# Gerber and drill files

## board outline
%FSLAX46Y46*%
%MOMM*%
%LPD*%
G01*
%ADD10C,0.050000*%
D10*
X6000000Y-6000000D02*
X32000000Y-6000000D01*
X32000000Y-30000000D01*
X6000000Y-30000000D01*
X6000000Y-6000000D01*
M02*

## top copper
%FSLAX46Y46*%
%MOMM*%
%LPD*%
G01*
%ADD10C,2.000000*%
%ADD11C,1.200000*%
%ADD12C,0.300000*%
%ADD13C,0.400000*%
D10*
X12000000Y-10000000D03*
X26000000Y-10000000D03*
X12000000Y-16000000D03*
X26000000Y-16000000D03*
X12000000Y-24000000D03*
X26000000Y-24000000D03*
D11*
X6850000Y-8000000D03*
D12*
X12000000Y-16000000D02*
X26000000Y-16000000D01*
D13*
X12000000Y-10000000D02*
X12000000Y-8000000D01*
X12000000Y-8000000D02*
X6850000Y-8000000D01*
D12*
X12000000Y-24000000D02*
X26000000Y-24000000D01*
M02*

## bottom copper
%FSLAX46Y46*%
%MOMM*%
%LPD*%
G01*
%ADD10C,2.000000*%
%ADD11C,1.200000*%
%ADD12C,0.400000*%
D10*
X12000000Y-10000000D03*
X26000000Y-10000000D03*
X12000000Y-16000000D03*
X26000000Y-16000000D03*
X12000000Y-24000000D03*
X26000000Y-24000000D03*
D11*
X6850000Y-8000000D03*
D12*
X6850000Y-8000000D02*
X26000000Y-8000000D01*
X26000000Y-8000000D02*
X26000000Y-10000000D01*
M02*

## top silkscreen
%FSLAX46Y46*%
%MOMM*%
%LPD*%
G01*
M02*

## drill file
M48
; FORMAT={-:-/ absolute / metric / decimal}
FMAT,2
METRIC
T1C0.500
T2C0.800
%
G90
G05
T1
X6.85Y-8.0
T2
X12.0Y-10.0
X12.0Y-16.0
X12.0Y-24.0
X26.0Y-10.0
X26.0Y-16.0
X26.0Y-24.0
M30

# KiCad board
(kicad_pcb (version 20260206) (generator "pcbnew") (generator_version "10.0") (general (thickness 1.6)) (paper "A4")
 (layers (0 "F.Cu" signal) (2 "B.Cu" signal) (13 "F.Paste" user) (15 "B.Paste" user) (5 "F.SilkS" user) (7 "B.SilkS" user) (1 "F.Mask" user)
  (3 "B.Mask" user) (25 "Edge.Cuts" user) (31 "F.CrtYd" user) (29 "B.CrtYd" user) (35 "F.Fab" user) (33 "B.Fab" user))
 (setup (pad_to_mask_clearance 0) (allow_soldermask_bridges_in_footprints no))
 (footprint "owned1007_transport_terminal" (layer "F.Cu") (at 12 10)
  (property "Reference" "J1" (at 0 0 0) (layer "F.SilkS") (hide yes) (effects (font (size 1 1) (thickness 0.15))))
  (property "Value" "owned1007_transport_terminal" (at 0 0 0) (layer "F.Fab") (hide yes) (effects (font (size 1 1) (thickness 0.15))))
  (pad "1" thru_hole circle (at 0 0) (size 2 2) (drill 0.8) (layers "*.Cu" "*.Mask") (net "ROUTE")))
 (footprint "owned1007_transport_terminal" (layer "F.Cu") (at 26 10)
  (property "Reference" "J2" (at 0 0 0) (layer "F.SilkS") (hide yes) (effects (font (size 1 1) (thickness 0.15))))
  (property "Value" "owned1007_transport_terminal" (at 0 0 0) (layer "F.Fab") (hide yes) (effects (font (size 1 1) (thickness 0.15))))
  (pad "1" thru_hole circle (at 0 0) (size 2 2) (drill 0.8) (layers "*.Cu" "*.Mask") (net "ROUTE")))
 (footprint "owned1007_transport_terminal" (layer "F.Cu") (at 12 16)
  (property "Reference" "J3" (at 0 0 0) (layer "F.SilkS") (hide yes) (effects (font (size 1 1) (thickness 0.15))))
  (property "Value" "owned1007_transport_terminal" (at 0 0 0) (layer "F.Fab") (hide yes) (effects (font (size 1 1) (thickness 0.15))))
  (pad "1" thru_hole circle (at 0 0) (size 2 2) (drill 0.8) (layers "*.Cu" "*.Mask") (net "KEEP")))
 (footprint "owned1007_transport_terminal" (layer "F.Cu") (at 26 16)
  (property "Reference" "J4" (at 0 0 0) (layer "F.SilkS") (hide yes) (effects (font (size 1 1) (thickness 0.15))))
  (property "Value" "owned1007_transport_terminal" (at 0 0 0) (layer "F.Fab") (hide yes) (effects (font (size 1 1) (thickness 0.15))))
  (pad "1" thru_hole circle (at 0 0) (size 2 2) (drill 0.8) (layers "*.Cu" "*.Mask") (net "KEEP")))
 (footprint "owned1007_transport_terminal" (layer "F.Cu") (at 12 24)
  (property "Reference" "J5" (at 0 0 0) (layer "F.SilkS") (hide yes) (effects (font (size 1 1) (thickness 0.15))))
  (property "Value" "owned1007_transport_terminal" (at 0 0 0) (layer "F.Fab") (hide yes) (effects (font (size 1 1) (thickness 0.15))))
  (pad "1" thru_hole circle (at 0 0) (size 2 2) (drill 0.8) (layers "*.Cu" "*.Mask") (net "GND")))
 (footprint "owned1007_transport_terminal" (layer "F.Cu") (at 26 24)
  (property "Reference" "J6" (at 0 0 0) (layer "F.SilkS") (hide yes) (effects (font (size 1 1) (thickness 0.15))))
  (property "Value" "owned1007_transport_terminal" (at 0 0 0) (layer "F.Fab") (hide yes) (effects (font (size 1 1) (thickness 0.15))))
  (pad "1" thru_hole circle (at 0 0) (size 2 2) (drill 0.8) (layers "*.Cu" "*.Mask") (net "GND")))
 (gr_rect (start 6 6) (end 32 30) (stroke (width 0.05) (type default)) (fill none) (layer "Edge.Cuts"))
 (segment (start 12 16) (end 26 16) (width 0.3) (layer "F.Cu") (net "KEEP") (locked yes))
 (segment (start 12 10) (end 12 8) (width 0.4) (layer "F.Cu") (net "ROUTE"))
 (segment (start 12 8) (end 6.85 8) (width 0.4) (layer "F.Cu") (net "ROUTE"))
 (segment (start 6.85 8) (end 26 8) (width 0.4) (layer "B.Cu") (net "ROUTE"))
 (segment (start 26 8) (end 26 10) (width 0.4) (layer "B.Cu") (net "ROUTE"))
 (via (at 6.85 8) (size 1.2) (drill 0.5) (layers "F.Cu" "B.Cu") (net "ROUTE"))
 (segment (start 12 24) (end 26 24) (width 0.3) (layer "F.Cu") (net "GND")))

